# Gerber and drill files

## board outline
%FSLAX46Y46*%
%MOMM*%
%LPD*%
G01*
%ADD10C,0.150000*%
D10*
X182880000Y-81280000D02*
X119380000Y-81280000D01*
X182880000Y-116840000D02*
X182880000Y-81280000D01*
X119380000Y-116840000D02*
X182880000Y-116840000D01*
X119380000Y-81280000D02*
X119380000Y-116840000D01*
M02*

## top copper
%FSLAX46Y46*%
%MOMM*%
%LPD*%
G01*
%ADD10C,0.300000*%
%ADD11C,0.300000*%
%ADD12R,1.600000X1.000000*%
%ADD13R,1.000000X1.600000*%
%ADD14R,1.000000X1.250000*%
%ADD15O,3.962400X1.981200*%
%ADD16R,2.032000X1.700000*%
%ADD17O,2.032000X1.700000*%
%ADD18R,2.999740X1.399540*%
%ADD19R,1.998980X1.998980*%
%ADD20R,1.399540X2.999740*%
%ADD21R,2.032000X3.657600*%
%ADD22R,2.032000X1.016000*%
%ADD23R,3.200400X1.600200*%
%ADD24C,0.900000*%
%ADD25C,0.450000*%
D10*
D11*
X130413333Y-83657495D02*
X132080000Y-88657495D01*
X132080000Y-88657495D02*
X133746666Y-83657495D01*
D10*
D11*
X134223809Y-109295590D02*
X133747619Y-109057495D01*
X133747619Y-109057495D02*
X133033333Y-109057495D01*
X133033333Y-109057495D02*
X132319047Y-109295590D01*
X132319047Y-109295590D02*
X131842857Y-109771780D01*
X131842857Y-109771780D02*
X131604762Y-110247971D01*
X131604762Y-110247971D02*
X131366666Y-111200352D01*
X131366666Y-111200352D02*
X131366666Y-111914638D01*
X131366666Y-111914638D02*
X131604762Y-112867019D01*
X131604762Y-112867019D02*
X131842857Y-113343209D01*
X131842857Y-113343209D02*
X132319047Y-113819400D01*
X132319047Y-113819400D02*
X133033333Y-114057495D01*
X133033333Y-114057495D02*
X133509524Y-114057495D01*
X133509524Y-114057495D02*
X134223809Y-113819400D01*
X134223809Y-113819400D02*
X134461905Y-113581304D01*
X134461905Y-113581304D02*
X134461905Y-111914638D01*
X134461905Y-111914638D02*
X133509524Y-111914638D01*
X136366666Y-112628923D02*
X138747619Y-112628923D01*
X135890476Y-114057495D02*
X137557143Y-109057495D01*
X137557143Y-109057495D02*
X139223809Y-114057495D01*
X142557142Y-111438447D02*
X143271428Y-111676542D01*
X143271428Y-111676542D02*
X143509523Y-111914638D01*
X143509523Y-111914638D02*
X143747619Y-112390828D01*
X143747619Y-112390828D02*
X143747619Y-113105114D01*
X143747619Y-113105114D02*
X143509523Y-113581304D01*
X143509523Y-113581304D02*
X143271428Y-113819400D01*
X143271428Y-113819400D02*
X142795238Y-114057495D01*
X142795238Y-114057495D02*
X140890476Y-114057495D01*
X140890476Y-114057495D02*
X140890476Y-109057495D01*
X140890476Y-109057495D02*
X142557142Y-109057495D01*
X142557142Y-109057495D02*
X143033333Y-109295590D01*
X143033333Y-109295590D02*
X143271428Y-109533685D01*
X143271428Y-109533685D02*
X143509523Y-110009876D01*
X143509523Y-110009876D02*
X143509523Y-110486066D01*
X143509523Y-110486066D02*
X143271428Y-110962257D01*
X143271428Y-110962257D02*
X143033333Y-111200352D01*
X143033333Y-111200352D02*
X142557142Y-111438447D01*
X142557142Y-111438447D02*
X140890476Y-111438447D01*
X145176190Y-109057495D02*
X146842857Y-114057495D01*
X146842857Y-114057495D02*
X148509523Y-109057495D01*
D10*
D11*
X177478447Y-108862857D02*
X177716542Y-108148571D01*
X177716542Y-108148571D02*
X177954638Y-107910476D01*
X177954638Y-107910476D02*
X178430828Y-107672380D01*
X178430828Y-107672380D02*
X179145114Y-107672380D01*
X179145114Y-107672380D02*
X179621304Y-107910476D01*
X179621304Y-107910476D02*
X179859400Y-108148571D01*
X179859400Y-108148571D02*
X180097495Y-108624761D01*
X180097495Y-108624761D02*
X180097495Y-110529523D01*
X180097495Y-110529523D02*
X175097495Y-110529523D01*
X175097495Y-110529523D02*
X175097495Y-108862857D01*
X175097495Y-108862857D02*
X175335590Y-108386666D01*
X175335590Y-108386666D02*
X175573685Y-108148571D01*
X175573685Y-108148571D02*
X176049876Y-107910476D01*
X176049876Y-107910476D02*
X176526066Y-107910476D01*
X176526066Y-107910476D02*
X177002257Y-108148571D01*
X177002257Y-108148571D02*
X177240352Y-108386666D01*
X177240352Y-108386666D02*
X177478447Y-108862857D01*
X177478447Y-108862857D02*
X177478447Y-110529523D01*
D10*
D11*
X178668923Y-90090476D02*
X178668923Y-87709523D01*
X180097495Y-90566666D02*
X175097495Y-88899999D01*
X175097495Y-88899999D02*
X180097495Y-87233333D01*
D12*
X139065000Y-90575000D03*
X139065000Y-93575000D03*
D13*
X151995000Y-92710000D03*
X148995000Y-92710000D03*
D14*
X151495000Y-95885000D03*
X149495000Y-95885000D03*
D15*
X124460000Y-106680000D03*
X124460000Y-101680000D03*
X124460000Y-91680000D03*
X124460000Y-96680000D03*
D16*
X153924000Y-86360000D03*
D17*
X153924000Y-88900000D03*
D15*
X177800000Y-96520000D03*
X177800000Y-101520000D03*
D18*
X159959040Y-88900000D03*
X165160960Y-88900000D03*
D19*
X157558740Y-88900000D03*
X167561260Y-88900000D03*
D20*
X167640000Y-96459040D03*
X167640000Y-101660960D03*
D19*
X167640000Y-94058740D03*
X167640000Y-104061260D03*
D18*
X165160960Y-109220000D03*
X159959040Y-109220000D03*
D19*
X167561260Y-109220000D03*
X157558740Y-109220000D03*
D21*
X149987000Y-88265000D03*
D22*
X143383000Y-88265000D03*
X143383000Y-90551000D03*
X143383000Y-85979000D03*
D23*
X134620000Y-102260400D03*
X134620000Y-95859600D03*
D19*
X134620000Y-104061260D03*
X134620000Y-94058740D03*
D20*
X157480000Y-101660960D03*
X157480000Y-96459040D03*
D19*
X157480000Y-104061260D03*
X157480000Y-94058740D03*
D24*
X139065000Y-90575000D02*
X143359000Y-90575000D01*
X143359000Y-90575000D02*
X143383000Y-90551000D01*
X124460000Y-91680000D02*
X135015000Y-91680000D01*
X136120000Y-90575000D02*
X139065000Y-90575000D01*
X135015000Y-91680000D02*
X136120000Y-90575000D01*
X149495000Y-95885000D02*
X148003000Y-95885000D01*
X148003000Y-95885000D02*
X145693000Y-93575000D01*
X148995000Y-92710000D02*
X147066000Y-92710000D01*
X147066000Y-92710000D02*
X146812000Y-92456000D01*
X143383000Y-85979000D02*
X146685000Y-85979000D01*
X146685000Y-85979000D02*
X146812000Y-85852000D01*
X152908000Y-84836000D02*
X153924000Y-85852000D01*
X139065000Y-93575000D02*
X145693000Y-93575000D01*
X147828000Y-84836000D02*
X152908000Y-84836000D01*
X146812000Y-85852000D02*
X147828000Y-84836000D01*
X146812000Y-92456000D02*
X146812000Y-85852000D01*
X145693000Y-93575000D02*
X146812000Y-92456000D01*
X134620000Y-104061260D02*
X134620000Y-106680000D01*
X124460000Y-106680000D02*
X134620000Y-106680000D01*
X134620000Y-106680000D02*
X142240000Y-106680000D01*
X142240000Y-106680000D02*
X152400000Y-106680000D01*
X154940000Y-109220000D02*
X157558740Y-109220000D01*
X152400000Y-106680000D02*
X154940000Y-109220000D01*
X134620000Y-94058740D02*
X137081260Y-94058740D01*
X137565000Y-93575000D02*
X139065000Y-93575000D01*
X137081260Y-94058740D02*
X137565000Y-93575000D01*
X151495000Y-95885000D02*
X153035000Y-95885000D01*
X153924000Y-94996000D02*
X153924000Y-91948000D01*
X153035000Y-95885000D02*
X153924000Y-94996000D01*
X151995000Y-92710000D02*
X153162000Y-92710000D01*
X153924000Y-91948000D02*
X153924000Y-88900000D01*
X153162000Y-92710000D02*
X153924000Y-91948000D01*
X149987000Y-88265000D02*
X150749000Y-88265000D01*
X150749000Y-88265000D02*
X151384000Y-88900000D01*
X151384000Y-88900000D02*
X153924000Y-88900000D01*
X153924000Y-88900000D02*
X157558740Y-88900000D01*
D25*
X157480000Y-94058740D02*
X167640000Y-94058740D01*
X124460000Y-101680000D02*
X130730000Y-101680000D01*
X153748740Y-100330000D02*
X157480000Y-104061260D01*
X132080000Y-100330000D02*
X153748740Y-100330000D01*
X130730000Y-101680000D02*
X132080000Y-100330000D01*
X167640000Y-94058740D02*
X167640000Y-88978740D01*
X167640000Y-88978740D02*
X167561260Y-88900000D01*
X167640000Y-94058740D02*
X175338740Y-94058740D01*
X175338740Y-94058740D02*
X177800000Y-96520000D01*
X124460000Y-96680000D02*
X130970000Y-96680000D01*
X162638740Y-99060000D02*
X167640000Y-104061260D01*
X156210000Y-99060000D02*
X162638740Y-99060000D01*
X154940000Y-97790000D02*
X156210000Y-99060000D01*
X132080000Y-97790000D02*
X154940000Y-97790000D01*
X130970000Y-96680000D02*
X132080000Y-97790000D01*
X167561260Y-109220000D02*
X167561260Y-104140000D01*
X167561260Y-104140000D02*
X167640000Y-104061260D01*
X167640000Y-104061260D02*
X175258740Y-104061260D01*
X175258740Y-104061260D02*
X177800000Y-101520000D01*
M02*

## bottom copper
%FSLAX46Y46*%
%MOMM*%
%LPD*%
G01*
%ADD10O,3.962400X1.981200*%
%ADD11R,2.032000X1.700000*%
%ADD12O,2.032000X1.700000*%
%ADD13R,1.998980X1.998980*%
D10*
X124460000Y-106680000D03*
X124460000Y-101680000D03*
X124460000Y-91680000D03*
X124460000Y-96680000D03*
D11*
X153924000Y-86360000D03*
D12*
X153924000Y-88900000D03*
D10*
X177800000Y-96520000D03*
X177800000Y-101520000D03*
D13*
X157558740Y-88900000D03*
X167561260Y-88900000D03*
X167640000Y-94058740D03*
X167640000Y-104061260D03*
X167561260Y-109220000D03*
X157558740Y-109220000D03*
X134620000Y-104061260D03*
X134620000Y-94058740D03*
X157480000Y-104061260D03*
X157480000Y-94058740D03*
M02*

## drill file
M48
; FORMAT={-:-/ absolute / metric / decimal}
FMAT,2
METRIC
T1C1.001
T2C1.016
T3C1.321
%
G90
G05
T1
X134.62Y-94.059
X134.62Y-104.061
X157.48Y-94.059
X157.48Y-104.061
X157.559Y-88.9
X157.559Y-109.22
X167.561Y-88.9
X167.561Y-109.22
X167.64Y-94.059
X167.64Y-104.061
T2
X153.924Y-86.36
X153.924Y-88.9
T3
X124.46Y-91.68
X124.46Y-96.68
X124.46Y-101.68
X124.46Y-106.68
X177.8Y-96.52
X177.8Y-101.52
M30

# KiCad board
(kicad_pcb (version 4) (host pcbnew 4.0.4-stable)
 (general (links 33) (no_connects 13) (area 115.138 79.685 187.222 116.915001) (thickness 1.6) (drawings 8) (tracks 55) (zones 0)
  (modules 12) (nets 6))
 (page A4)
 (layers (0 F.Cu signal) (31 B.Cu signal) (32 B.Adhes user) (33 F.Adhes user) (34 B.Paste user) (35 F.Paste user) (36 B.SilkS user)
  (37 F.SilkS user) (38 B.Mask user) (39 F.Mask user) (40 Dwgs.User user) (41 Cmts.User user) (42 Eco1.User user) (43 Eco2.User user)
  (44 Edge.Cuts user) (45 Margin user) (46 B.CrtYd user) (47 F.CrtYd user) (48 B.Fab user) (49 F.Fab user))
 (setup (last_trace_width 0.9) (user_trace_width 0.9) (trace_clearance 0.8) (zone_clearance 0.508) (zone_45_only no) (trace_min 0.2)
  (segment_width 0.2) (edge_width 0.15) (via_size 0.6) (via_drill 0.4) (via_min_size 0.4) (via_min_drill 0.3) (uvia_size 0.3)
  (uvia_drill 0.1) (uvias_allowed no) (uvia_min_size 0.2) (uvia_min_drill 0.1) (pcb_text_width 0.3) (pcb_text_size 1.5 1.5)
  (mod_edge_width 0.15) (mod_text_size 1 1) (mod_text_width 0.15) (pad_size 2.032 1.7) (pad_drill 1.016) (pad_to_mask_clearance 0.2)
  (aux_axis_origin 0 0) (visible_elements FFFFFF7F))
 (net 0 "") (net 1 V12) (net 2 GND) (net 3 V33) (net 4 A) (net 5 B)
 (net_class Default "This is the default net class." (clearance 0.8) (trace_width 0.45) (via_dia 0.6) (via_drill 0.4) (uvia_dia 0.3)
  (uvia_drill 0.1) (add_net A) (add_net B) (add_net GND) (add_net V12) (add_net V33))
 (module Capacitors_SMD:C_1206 (layer F.Cu) (at 139.065 92.075 270)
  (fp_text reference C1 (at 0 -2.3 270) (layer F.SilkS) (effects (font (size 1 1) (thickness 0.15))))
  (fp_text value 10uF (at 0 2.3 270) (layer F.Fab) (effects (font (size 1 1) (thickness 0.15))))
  (pad 1 smd rect (at -1.5 0 270) (size 1 1.6) (layers F.Cu F.Paste F.Mask) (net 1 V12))
  (pad 2 smd rect (at 1.5 0 270) (size 1 1.6) (layers F.Cu F.Paste F.Mask) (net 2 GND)))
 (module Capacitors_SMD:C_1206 (layer F.Cu) (at 150.495 92.71 180)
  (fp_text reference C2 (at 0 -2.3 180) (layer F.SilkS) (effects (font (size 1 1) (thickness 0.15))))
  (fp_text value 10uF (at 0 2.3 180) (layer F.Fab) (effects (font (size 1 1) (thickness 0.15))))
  (pad 1 smd rect (at -1.5 0 180) (size 1 1.6) (layers F.Cu F.Paste F.Mask) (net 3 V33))
  (pad 2 smd rect (at 1.5 0 180) (size 1 1.6) (layers F.Cu F.Paste F.Mask) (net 2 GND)))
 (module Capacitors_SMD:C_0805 (layer F.Cu) (at 150.495 95.885 180)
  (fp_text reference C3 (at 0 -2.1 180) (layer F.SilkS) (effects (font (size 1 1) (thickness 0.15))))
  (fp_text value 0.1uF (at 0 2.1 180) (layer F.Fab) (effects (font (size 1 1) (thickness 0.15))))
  (pad 1 smd rect (at -1 0 180) (size 1 1.25) (layers F.Cu F.Paste F.Mask) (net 3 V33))
  (pad 2 smd rect (at 1 0 180) (size 1 1.25) (layers F.Cu F.Paste F.Mask) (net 2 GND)))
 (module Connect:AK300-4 (layer B.Cu) (at 124.46 106.68 90)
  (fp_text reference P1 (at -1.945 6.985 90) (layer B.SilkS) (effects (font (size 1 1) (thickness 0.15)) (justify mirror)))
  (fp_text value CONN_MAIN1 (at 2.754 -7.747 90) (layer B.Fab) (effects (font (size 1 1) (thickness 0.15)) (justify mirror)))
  (pad 1 thru_hole oval (at 0 0 90) (size 1.9812 3.9624) (drill 1.3208) (layers *.Cu B.Paste B.SilkS B.Mask) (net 2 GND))
  (pad 2 thru_hole oval (at 5 0 90) (size 1.9812 3.9624) (drill 1.3208) (layers *.Cu B.Paste B.SilkS B.Mask) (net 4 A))
  (pad 4 thru_hole oval (at 15 0 90) (size 1.9812 3.9624) (drill 1.3208) (layers *.Cu B.Paste B.SilkS B.Mask) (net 1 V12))
  (pad 3 thru_hole oval (at 10 0 90) (size 1.9812 3.9624) (drill 1.3208) (layers *.Cu *.Mask B.SilkS) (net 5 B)))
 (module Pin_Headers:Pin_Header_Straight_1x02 (layer B.Cu) (at 153.924 86.36 180)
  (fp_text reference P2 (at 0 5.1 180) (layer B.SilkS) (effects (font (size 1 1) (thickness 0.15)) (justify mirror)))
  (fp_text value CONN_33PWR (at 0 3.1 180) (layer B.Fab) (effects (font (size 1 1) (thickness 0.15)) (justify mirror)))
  (pad 1 thru_hole rect (at 0 0 180) (size 2.032 1.7) (drill 1.016) (layers *.Cu *.Mask B.SilkS) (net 2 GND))
  (pad 2 thru_hole oval (at 0 -2.54 180) (size 2.032 1.7) (drill 1.016) (layers *.Cu *.Mask B.SilkS) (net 3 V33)))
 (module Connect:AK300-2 (layer B.Cu) (at 177.8 96.52 270)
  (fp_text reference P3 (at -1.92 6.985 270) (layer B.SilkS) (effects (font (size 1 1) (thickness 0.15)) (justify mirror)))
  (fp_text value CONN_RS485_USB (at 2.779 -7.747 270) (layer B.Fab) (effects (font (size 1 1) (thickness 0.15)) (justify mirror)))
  (pad 1 thru_hole oval (at 0 0 270) (size 1.9812 3.9624) (drill 1.3208) (layers *.Cu B.Paste B.SilkS B.Mask) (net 4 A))
  (pad 2 thru_hole oval (at 5 0 270) (size 1.9812 3.9624) (drill 1.3208) (layers *.Cu B.Paste B.SilkS B.Mask) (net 5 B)))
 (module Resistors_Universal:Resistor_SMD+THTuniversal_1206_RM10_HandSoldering (layer F.Cu) (at 162.56 88.9)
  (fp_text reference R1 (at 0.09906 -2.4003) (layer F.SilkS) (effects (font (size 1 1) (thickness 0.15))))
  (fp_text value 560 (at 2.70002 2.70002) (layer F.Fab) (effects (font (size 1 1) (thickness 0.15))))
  (pad 1 smd rect (at -2.60096 0) (size 2.99974 1.39954) (layers F.Cu F.Paste F.Mask) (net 3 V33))
  (pad 2 smd rect (at 2.60096 0) (size 2.99974 1.39954) (layers F.Cu F.Paste F.Mask) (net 4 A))
  (pad 1 thru_hole rect (at -5.00126 0) (size 1.99898 1.99898) (drill 1.00076) (layers *.Cu *.Mask F.SilkS) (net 3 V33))
  (pad 2 thru_hole rect (at 5.00126 0) (size 1.99898 1.99898) (drill 1.00076) (layers *.Cu *.Mask F.SilkS) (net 4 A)))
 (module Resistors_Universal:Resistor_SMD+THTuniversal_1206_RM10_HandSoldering (layer F.Cu) (at 167.64 99.06 270)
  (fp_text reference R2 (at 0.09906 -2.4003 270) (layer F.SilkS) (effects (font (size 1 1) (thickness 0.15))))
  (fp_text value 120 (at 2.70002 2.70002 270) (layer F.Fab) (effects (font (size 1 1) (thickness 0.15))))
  (pad 1 smd rect (at -2.60096 0 270) (size 2.99974 1.39954) (layers F.Cu F.Paste F.Mask) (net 4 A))
  (pad 2 smd rect (at 2.60096 0 270) (size 2.99974 1.39954) (layers F.Cu F.Paste F.Mask) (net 5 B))
  (pad 1 thru_hole rect (at -5.00126 0 270) (size 1.99898 1.99898) (drill 1.00076) (layers *.Cu *.Mask F.SilkS) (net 4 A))
  (pad 2 thru_hole rect (at 5.00126 0 270) (size 1.99898 1.99898) (drill 1.00076) (layers *.Cu *.Mask F.SilkS) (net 5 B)))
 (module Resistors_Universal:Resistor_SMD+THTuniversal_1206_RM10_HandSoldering (layer F.Cu) (at 162.56 109.22 180)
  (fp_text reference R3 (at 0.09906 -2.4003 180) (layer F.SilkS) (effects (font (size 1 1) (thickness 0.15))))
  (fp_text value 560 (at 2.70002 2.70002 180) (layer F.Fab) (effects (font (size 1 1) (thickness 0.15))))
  (pad 1 smd rect (at -2.60096 0 180) (size 2.99974 1.39954) (layers F.Cu F.Paste F.Mask) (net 5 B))
  (pad 2 smd rect (at 2.60096 0 180) (size 2.99974 1.39954) (layers F.Cu F.Paste F.Mask) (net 2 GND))
  (pad 1 thru_hole rect (at -5.00126 0 180) (size 1.99898 1.99898) (drill 1.00076) (layers *.Cu *.Mask F.SilkS) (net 5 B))
  (pad 2 thru_hole rect (at 5.00126 0 180) (size 1.99898 1.99898) (drill 1.00076) (layers *.Cu *.Mask F.SilkS) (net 2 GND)))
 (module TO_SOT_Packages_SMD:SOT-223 (layer F.Cu) (at 146.685 88.265 270)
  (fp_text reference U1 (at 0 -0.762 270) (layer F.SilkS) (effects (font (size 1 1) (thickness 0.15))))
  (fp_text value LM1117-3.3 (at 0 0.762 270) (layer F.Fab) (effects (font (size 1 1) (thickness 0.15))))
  (pad 4 smd rect (at 0 -3.302 270) (size 3.6576 2.032) (layers F.Cu F.Paste F.Mask) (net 3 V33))
  (pad 2 smd rect (at 0 3.302 270) (size 1.016 2.032) (layers F.Cu F.Paste F.Mask) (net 3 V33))
  (pad 3 smd rect (at 2.286 3.302 270) (size 1.016 2.032) (layers F.Cu F.Paste F.Mask) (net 1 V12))
  (pad 1 smd rect (at -2.286 3.302 270) (size 1.016 2.032) (layers F.Cu F.Paste F.Mask) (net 2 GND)))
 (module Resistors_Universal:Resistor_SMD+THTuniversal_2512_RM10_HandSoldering (layer F.Cu) (at 134.62 99.06 90)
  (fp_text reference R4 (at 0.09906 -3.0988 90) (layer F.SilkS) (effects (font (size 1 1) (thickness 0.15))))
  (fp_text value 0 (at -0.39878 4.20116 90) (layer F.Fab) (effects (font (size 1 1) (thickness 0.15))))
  (pad 1 smd rect (at -3.2004 0 90) (size 1.6002 3.2004) (layers F.Cu F.Paste F.Mask) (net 2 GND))
  (pad 2 smd rect (at 3.2004 0 90) (size 1.6002 3.2004) (layers F.Cu F.Paste F.Mask) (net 2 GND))
  (pad 1 thru_hole rect (at -5.00126 0 270) (size 1.99898 1.99898) (drill 1.00076) (layers *.Cu *.Mask F.SilkS) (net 2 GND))
  (pad 2 thru_hole rect (at 5.00126 0 270) (size 1.99898 1.99898) (drill 1.00076) (layers *.Cu *.Mask F.SilkS) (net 2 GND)))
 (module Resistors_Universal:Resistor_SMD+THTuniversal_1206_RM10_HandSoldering (layer F.Cu) (at 157.48 99.06 90)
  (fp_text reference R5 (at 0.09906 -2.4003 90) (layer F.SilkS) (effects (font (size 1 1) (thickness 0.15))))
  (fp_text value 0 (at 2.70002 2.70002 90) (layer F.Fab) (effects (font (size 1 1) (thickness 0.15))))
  (pad 1 smd rect (at -2.60096 0 90) (size 2.99974 1.39954) (layers F.Cu F.Paste F.Mask) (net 4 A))
  (pad 2 smd rect (at 2.60096 0 90) (size 2.99974 1.39954) (layers F.Cu F.Paste F.Mask) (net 4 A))
  (pad 1 thru_hole rect (at -5.00126 0 90) (size 1.99898 1.99898) (drill 1.00076) (layers *.Cu *.Mask F.SilkS) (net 4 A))
  (pad 2 thru_hole rect (at 5.00126 0 90) (size 1.99898 1.99898) (drill 1.00076) (layers *.Cu *.Mask F.SilkS) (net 4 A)))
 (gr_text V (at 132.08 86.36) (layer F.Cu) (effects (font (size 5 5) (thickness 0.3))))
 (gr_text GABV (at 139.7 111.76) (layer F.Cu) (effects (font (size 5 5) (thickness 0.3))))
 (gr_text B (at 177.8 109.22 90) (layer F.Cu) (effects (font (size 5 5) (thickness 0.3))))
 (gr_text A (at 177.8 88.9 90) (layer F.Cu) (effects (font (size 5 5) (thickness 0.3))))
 (gr_line (start 182.88 81.28) (end 119.38 81.28) (angle 90) (layer Edge.Cuts) (width 0.15))
 (gr_line (start 182.88 116.84) (end 182.88 81.28) (angle 90) (layer Edge.Cuts) (width 0.15))
 (gr_line (start 119.38 116.84) (end 182.88 116.84) (angle 90) (layer Edge.Cuts) (width 0.15))
 (gr_line (start 119.38 81.28) (end 119.38 116.84) (angle 90) (layer Edge.Cuts) (width 0.15))
 (segment (start 139.065 90.575) (end 143.359 90.575) (width 0.9) (layer F.Cu) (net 1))
 (segment (start 143.359 90.575) (end 143.383 90.551) (width 0.9) (layer F.Cu) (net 1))
 (segment (start 124.46 91.68) (end 135.015 91.68) (width 0.9) (layer F.Cu) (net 1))
 (segment (start 136.12 90.575) (end 139.065 90.575) (width 0.9) (layer F.Cu) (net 1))
 (segment (start 135.015 91.68) (end 136.12 90.575) (width 0.9) (layer F.Cu) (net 1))
 (segment (start 149.495 95.885) (end 148.003 95.885) (width 0.9) (layer F.Cu) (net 2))
 (segment (start 148.003 95.885) (end 145.693 93.575) (width 0.9) (layer F.Cu) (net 2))
 (segment (start 148.995 92.71) (end 147.066 92.71) (width 0.9) (layer F.Cu) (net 2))
 (segment (start 147.066 92.71) (end 146.812 92.456) (width 0.9) (layer F.Cu) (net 2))
 (segment (start 143.383 85.979) (end 146.685 85.979) (width 0.9) (layer F.Cu) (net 2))
 (segment (start 146.685 85.979) (end 146.812 85.852) (width 0.9) (layer F.Cu) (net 2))
 (segment (start 152.908 84.836) (end 153.924 85.852) (width 0.9) (layer F.Cu) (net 2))
 (segment (start 139.065 93.575) (end 145.693 93.575) (width 0.9) (layer F.Cu) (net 2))
 (segment (start 147.828 84.836) (end 152.908 84.836) (width 0.9) (layer F.Cu) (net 2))
 (segment (start 146.812 85.852) (end 147.828 84.836) (width 0.9) (layer F.Cu) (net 2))
 (segment (start 146.812 92.456) (end 146.812 85.852) (width 0.9) (layer F.Cu) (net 2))
 (segment (start 145.693 93.575) (end 146.812 92.456) (width 0.9) (layer F.Cu) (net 2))
 (segment (start 134.62 104.06126) (end 134.62 106.68) (width 0.9) (layer F.Cu) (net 2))
 (segment (start 124.46 106.68) (end 134.62 106.68) (width 0.9) (layer F.Cu) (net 2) (status 10))
 (segment (start 134.62 106.68) (end 142.24 106.68) (width 0.9) (layer F.Cu) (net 2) (status 10))
 (segment (start 142.24 106.68) (end 152.4 106.68) (width 0.9) (layer F.Cu) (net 2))
 (segment (start 154.94 109.22) (end 157.55874 109.22) (width 0.9) (layer F.Cu) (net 2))
 (segment (start 152.4 106.68) (end 154.94 109.22) (width 0.9) (layer F.Cu) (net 2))
 (segment (start 134.62 94.05874) (end 137.08126 94.05874) (width 0.9) (layer F.Cu) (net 2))
 (segment (start 137.565 93.575) (end 139.065 93.575) (width 0.9) (layer F.Cu) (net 2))
 (segment (start 137.08126 94.05874) (end 137.565 93.575) (width 0.9) (layer F.Cu) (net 2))
 (segment (start 151.495 95.885) (end 153.035 95.885) (width 0.9) (layer F.Cu) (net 3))
 (segment (start 153.924 94.996) (end 153.924 91.948) (width 0.9) (layer F.Cu) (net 3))
 (segment (start 153.035 95.885) (end 153.924 94.996) (width 0.9) (layer F.Cu) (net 3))
 (segment (start 151.995 92.71) (end 153.162 92.71) (width 0.9) (layer F.Cu) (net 3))
 (segment (start 153.924 91.948) (end 153.924 88.9) (width 0.9) (layer F.Cu) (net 3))
 (segment (start 153.162 92.71) (end 153.924 91.948) (width 0.9) (layer F.Cu) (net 3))
 (segment (start 149.987 88.265) (end 150.749 88.265) (width 0.9) (layer F.Cu) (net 3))
 (segment (start 150.749 88.265) (end 151.384 88.9) (width 0.9) (layer F.Cu) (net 3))
 (segment (start 151.384 88.9) (end 153.924 88.9) (width 0.9) (layer F.Cu) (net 3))
 (segment (start 153.924 88.9) (end 157.55874 88.9) (width 0.9) (layer F.Cu) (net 3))
 (segment (start 157.48 94.05874) (end 167.64 94.05874) (width 0.45) (layer F.Cu) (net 4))
 (segment (start 124.46 101.68) (end 130.73 101.68) (width 0.45) (layer F.Cu) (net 4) (status 10))
 (segment (start 153.74874 100.33) (end 157.48 104.06126) (width 0.45) (layer F.Cu) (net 4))
 (segment (start 132.08 100.33) (end 153.74874 100.33) (width 0.45) (layer F.Cu) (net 4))
 (segment (start 130.73 101.68) (end 132.08 100.33) (width 0.45) (layer F.Cu) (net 4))
 (segment (start 167.64 94.05874) (end 167.64 88.97874) (width 0.45) (layer F.Cu) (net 4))
 (segment (start 167.64 88.97874) (end 167.56126 88.9) (width 0.45) (layer F.Cu) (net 4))
 (segment (start 167.64 94.05874) (end 175.33874 94.05874) (width 0.45) (layer F.Cu) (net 4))
 (segment (start 175.33874 94.05874) (end 177.8 96.52) (width 0.45) (layer F.Cu) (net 4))
 (segment (start 124.46 96.68) (end 130.97 96.68) (width 0.45) (layer F.Cu) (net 5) (status 10))
 (segment (start 162.63874 99.06) (end 167.64 104.06126) (width 0.45) (layer F.Cu) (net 5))
 (segment (start 156.21 99.06) (end 162.63874 99.06) (width 0.45) (layer F.Cu) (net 5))
 (segment (start 154.94 97.79) (end 156.21 99.06) (width 0.45) (layer F.Cu) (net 5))
 (segment (start 132.08 97.79) (end 154.94 97.79) (width 0.45) (layer F.Cu) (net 5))
 (segment (start 130.97 96.68) (end 132.08 97.79) (width 0.45) (layer F.Cu) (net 5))
 (segment (start 167.56126 109.22) (end 167.56126 104.14) (width 0.45) (layer F.Cu) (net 5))
 (segment (start 167.56126 104.14) (end 167.64 104.06126) (width 0.45) (layer F.Cu) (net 5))
 (segment (start 167.64 104.06126) (end 175.25874 104.06126) (width 0.45) (layer F.Cu) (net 5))
 (segment (start 175.25874 104.06126) (end 177.8 101.52) (width 0.45) (layer F.Cu) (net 5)))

